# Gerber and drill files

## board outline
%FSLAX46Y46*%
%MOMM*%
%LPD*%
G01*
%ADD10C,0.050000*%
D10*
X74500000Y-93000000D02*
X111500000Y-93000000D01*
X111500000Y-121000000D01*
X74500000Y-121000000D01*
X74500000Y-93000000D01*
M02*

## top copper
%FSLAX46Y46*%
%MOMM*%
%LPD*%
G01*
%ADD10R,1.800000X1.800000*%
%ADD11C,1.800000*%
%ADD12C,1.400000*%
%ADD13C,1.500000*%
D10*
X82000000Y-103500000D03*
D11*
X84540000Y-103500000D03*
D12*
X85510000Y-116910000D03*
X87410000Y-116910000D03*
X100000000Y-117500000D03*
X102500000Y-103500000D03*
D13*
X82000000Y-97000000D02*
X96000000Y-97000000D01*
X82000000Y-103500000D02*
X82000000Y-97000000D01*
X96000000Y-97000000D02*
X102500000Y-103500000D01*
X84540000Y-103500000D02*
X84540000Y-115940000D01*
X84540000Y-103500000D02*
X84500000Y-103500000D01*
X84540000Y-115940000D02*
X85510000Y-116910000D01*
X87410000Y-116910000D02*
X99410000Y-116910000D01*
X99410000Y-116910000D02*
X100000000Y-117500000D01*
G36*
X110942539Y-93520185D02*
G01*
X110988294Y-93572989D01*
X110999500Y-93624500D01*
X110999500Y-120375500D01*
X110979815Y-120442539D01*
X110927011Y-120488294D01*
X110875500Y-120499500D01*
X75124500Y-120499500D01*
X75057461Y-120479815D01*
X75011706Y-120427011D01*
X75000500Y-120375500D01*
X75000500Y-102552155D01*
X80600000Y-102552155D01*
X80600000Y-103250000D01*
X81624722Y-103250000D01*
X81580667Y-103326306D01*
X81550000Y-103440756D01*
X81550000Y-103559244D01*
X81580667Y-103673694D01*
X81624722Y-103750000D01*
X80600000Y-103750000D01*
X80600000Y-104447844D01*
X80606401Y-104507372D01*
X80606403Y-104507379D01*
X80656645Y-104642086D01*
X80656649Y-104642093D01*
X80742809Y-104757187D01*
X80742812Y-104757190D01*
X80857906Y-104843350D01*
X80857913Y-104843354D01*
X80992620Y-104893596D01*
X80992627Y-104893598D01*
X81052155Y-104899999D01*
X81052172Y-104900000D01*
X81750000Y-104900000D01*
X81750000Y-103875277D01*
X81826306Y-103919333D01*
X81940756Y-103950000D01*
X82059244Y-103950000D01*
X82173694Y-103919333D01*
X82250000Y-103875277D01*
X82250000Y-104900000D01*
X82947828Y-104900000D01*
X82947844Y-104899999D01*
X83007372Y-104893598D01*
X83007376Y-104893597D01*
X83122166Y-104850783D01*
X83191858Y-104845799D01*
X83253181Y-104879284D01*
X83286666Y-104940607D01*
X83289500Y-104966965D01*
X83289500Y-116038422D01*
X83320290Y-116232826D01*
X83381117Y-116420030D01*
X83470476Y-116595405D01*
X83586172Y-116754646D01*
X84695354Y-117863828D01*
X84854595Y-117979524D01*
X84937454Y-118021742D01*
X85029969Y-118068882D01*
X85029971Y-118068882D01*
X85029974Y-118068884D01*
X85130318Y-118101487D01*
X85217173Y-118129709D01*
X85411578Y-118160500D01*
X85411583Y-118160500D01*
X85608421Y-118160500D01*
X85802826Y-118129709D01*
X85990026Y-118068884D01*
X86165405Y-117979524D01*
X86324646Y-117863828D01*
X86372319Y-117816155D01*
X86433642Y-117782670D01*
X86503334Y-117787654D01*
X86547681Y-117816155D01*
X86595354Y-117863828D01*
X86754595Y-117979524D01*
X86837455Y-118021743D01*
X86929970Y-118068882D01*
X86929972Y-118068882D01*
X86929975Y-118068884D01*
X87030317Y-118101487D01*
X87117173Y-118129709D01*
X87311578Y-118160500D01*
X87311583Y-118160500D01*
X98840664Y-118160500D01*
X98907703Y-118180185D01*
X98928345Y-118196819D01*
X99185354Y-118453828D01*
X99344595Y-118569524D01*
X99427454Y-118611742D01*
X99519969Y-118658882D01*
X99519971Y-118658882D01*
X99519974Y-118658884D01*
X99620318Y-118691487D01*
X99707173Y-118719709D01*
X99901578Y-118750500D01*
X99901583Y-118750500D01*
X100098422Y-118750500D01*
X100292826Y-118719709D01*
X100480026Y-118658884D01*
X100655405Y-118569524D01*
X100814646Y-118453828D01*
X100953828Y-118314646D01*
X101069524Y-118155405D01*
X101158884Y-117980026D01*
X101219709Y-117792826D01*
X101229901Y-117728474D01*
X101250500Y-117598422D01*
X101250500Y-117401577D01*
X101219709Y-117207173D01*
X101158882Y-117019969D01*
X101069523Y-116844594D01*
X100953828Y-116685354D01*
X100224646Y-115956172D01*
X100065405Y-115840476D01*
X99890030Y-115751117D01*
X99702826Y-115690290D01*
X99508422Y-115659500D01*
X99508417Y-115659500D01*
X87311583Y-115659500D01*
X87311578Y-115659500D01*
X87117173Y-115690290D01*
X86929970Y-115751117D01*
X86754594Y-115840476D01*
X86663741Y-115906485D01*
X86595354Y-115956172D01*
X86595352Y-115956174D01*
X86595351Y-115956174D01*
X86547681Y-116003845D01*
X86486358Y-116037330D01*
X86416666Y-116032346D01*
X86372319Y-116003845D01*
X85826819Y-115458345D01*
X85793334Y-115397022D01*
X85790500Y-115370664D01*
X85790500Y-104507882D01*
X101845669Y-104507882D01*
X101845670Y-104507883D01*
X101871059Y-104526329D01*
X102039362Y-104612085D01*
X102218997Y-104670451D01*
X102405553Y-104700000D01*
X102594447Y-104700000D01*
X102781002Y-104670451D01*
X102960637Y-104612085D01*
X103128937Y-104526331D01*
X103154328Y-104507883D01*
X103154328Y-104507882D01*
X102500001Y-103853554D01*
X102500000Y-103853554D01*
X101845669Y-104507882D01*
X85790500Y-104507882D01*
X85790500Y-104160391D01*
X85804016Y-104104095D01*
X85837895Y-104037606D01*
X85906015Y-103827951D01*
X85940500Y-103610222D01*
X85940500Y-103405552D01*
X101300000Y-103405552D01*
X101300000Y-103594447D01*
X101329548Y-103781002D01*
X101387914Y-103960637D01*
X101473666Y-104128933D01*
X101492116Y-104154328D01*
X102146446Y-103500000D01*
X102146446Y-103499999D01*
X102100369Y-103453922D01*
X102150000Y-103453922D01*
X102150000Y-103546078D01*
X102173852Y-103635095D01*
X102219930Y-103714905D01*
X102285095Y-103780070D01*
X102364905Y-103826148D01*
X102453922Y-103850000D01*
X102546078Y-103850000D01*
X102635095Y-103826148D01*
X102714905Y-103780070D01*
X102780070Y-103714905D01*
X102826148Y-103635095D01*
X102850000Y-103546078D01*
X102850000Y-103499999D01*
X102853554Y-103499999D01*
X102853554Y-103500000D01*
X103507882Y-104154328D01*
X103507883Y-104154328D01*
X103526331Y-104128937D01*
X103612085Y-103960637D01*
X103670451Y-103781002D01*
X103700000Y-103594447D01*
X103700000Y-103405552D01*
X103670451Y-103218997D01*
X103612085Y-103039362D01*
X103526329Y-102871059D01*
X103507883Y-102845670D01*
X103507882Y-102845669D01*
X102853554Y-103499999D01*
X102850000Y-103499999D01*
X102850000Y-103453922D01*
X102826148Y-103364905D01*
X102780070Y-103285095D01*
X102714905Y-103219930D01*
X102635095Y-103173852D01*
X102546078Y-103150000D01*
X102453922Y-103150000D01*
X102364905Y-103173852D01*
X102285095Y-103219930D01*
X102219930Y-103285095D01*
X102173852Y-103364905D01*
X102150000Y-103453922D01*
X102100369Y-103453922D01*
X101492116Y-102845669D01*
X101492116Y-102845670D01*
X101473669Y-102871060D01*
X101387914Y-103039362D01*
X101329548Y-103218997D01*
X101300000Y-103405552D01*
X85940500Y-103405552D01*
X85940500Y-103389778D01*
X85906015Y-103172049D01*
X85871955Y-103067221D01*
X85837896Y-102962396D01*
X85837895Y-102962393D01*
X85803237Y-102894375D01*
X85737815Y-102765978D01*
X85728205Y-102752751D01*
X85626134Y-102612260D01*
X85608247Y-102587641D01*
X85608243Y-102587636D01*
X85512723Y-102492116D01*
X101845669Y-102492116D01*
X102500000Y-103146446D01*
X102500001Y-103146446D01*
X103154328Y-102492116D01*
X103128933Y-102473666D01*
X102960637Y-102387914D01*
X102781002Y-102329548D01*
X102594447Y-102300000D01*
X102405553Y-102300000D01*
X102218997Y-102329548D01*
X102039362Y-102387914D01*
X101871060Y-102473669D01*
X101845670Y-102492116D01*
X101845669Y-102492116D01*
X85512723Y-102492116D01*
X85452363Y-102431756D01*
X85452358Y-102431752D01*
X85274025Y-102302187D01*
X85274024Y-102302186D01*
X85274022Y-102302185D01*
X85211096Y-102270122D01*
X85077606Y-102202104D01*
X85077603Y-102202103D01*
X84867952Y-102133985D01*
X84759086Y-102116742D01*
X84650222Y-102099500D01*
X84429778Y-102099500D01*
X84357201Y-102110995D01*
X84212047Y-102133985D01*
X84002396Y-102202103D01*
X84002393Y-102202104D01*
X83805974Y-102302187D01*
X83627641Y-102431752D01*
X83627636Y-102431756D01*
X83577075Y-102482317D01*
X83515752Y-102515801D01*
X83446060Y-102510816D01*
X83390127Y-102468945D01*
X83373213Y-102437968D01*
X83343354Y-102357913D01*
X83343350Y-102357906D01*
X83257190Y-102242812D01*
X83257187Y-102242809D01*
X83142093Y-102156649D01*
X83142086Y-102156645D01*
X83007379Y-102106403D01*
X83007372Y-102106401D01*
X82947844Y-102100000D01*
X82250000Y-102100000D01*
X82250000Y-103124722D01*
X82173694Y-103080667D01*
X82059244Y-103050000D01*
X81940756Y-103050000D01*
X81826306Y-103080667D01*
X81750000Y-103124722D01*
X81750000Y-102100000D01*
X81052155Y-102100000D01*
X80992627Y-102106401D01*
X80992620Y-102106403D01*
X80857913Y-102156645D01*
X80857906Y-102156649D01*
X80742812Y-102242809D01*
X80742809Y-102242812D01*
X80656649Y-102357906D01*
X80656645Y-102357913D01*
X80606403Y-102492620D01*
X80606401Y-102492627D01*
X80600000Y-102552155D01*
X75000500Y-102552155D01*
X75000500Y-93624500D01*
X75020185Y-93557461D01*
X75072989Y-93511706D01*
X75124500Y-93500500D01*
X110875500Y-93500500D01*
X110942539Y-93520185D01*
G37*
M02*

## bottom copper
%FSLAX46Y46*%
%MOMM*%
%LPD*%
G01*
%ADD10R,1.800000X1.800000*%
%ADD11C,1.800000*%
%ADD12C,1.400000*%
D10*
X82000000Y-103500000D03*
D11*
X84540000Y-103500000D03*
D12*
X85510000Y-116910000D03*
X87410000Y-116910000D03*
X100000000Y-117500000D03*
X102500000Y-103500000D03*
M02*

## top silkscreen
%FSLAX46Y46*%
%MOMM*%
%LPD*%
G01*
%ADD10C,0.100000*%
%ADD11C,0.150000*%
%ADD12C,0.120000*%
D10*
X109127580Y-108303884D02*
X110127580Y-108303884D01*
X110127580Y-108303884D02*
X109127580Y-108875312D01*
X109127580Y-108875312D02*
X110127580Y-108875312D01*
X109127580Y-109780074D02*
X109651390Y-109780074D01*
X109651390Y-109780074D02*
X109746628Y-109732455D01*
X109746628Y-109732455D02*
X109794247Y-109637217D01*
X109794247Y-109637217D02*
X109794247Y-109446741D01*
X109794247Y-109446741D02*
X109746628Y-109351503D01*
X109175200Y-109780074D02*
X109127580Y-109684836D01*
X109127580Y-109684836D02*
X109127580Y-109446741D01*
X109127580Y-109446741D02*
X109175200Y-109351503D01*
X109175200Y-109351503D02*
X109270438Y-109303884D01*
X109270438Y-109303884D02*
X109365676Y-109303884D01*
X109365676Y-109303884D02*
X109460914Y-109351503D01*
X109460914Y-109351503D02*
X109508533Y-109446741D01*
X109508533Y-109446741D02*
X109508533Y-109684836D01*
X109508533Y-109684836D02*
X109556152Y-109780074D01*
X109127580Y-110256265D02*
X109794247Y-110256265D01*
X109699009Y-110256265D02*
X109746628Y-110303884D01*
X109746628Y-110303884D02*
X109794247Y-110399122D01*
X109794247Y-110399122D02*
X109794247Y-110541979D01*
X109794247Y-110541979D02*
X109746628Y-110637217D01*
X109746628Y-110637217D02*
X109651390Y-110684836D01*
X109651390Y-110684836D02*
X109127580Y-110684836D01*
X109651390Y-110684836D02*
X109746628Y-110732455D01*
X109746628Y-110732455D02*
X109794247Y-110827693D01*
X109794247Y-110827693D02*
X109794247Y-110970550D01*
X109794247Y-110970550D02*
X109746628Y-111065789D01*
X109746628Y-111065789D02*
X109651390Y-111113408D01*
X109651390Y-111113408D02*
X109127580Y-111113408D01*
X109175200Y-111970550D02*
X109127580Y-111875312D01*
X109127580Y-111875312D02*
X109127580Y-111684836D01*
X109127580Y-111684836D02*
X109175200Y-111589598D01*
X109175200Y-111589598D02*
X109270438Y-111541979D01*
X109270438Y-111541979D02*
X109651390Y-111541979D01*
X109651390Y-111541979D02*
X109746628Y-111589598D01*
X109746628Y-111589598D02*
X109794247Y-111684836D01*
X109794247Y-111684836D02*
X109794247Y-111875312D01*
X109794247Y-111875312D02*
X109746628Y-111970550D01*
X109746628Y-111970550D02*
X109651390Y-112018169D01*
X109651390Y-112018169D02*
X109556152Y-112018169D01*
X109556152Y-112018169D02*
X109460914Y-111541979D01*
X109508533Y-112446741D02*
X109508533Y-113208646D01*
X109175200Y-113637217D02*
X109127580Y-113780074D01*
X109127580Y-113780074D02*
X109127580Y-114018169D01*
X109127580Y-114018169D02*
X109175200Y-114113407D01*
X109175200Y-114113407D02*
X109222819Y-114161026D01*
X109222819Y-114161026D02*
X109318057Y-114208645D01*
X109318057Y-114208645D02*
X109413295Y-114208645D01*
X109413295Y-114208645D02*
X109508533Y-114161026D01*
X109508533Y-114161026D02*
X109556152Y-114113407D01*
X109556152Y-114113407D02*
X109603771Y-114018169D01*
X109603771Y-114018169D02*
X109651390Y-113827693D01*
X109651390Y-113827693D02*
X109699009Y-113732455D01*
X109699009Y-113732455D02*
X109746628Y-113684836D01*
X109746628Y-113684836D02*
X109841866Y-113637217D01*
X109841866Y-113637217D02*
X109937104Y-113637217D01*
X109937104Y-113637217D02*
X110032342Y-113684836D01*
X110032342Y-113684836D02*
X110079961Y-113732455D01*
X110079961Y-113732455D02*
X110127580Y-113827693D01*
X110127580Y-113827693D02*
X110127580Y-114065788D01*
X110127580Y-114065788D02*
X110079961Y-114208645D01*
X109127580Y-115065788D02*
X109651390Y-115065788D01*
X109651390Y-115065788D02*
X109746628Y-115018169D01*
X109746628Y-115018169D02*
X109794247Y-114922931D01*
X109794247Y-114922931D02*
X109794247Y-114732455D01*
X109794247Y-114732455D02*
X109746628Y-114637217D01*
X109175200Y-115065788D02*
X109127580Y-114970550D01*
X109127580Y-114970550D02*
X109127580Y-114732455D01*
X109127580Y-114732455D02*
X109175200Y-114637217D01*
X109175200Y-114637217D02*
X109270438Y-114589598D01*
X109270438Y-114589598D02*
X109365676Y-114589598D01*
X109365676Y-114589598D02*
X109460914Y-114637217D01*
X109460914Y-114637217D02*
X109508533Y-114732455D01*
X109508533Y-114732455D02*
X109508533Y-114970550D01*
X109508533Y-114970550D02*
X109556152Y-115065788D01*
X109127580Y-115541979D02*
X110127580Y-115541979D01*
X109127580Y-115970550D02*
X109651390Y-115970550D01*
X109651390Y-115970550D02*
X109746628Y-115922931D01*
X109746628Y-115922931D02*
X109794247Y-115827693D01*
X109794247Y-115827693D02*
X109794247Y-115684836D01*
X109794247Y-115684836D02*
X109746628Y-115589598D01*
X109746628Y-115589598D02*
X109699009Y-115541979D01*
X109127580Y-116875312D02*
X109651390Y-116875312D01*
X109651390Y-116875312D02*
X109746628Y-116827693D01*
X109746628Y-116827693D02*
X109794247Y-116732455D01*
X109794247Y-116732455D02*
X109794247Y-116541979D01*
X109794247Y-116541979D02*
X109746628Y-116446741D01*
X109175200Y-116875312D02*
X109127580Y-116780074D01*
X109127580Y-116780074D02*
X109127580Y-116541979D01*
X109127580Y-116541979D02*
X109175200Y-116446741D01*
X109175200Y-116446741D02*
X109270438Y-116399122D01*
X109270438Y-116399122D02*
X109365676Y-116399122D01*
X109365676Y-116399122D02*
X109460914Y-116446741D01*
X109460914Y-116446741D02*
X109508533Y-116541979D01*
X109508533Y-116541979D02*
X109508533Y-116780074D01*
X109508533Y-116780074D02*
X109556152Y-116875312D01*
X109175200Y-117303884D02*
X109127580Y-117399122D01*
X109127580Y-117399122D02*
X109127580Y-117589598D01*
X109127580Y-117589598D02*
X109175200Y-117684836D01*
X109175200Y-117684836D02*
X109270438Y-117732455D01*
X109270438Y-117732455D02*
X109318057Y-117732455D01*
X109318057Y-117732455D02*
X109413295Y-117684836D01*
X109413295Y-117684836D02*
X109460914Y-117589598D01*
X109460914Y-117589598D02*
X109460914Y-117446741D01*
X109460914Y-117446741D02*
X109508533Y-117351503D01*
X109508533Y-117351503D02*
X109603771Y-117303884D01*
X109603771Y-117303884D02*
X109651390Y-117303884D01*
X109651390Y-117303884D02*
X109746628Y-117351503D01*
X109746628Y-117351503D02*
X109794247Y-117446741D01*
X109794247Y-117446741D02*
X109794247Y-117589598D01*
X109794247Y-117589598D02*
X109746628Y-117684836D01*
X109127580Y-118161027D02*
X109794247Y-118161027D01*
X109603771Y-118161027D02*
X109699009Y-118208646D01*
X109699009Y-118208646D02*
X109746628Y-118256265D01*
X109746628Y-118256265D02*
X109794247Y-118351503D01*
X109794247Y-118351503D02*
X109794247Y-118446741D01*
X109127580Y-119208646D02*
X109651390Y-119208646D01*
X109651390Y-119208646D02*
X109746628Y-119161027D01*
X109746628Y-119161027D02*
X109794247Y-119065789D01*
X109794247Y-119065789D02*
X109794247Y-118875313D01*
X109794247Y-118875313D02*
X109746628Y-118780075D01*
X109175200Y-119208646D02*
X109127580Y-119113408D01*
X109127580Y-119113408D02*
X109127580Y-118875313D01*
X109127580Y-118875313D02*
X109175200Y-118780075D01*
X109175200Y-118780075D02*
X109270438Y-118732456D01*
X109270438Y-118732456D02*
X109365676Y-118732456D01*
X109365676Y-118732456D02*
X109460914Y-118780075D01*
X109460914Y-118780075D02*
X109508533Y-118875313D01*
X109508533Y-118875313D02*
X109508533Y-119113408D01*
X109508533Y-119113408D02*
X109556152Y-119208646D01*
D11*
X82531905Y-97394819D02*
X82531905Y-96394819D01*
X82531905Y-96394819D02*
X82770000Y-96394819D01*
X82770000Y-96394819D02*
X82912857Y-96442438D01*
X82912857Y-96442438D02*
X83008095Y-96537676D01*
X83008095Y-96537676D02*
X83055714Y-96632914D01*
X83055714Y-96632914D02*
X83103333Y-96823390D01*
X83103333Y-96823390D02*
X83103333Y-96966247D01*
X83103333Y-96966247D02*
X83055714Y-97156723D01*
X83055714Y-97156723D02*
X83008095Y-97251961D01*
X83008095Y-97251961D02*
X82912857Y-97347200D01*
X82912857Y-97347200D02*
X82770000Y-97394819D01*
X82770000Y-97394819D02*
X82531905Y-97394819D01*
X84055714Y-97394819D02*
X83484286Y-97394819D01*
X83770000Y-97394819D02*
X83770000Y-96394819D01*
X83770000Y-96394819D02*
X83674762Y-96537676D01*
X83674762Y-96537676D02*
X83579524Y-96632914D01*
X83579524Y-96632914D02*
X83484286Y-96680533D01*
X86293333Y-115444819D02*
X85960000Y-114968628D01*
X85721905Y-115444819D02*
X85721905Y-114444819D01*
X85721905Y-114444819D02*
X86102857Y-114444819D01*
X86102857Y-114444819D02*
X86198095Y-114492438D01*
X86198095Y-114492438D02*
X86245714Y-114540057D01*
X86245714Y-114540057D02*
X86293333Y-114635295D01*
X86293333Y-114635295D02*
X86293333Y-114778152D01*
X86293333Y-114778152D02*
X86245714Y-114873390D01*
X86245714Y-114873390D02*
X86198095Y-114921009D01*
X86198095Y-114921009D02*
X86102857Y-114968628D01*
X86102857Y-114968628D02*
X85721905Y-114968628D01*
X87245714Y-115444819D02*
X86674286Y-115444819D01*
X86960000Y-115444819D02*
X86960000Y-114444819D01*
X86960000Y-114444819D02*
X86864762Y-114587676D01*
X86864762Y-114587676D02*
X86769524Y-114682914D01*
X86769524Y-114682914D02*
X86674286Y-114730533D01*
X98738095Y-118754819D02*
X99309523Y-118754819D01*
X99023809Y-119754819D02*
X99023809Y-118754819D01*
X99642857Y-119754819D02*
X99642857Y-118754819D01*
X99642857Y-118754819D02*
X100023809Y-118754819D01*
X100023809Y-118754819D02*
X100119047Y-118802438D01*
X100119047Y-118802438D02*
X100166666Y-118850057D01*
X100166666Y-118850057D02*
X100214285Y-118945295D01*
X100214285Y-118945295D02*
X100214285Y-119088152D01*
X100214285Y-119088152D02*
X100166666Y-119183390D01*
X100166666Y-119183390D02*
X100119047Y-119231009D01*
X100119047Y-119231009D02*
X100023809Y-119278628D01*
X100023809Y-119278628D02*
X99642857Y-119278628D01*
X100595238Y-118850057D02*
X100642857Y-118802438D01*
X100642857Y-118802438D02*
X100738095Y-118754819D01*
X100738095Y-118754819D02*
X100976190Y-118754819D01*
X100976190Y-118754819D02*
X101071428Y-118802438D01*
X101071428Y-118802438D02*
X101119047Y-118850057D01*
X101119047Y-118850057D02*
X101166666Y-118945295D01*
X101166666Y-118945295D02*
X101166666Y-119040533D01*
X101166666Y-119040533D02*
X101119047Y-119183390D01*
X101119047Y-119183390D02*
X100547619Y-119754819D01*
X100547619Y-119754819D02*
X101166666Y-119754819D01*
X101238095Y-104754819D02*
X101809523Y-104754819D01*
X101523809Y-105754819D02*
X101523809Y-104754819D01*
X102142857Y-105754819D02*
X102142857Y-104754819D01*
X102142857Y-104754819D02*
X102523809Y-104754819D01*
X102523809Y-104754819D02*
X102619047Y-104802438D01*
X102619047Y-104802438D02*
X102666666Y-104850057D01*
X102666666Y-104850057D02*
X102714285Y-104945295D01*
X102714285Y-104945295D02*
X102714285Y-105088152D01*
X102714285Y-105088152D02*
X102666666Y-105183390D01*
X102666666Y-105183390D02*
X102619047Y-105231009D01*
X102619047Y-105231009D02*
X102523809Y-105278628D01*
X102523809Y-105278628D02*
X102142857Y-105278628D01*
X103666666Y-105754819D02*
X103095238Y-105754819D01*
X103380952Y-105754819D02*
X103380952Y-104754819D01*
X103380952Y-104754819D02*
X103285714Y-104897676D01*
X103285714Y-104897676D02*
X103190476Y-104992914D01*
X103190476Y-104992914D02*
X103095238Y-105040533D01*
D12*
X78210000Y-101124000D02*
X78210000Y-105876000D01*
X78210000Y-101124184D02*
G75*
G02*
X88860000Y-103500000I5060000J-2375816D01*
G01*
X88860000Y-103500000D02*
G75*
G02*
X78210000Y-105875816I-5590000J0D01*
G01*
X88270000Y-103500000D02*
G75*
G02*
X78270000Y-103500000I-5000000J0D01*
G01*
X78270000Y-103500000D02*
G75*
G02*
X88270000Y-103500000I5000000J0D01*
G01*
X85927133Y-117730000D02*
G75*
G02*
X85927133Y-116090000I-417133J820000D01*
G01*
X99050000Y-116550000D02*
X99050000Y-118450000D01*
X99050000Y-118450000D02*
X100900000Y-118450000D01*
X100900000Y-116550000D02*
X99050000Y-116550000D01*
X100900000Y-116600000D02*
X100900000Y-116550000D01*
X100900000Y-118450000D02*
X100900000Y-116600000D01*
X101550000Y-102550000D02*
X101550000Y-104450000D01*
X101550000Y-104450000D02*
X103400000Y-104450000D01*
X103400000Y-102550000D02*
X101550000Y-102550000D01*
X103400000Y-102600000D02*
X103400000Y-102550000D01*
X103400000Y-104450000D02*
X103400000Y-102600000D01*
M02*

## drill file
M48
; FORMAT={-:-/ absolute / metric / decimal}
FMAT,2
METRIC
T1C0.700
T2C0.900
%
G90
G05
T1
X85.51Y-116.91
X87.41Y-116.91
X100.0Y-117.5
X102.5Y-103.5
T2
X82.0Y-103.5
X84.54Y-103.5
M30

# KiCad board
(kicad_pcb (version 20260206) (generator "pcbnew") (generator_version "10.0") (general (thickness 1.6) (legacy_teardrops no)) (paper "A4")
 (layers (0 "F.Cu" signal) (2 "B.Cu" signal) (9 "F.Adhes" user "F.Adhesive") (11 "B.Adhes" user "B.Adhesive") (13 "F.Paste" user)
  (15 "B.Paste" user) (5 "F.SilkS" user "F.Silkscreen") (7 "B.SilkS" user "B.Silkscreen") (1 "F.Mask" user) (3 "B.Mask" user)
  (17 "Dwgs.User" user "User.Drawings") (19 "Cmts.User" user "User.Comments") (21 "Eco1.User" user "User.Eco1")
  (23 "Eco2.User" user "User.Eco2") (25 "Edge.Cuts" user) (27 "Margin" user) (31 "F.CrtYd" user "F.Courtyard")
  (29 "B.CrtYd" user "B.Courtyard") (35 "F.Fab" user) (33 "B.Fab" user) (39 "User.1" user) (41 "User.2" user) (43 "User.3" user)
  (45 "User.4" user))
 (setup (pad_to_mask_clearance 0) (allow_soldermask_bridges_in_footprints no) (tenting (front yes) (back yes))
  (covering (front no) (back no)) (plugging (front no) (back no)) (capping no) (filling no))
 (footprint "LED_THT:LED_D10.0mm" (layer "F.Cu") (at 82 103.5)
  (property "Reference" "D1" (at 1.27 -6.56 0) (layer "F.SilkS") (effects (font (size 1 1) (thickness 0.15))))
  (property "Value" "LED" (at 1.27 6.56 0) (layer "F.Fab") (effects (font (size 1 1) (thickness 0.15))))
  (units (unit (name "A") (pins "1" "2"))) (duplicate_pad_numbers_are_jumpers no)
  (fp_line (start -3.79 -2.376) (end -3.79 2.376) (stroke (width 0.12) (type solid)) (layer "F.SilkS"))
  (fp_arc (start -3.79 -2.375816) (mid 2.487107 -5.455891) (end 6.86 0) (stroke (width 0.12) (type solid)) (layer "F.SilkS"))
  (fp_arc (start 6.86 0) (mid 2.487107 5.455891) (end -3.79 2.375816) (stroke (width 0.12) (type solid)) (layer "F.SilkS"))
  (fp_circle (center 1.27 0) (end 6.27 0) (stroke (width 0.12) (type solid)) (fill no) (layer "F.SilkS"))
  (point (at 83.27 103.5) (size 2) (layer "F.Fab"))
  (pad "1" thru_hole rect (at 0 0) (size 1.8 1.8) (drill 0.9) (layers "*.Cu" "*.Mask") (remove_unused_layers no) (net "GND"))
  (pad "2" thru_hole circle (at 2.54 0) (size 1.8 1.8) (drill 0.9) (layers "*.Cu" "*.Mask") (remove_unused_layers no) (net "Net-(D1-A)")))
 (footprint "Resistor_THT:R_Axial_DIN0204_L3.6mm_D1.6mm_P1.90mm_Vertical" (layer "F.Cu") (at 85.51 116.91)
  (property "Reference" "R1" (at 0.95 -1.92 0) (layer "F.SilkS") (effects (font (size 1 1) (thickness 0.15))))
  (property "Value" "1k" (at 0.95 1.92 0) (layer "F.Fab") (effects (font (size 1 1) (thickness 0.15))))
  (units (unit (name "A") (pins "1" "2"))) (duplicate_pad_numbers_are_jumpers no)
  (fp_arc (start 0.417133 0.82) (mid -0.92 0) (end 0.417133 -0.82) (stroke (width 0.12) (type solid)) (layer "F.SilkS"))
  (pad "1" thru_hole circle (at 0 0) (size 1.4 1.4) (drill 0.7) (layers "*.Cu" "*.Mask") (remove_unused_layers no) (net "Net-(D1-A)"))
  (pad "2" thru_hole circle (at 1.9 0) (size 1.4 1.4) (drill 0.7) (layers "*.Cu" "*.Mask") (remove_unused_layers no) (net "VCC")))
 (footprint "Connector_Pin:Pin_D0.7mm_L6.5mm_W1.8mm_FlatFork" (layer "F.Cu") (at 100 117.5)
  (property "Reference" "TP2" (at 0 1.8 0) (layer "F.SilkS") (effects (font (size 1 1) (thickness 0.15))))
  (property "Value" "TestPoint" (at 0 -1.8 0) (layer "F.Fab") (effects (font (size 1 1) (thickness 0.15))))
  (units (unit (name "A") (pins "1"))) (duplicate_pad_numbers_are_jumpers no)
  (fp_line (start -0.95 -0.95) (end -0.95 0.95) (stroke (width 0.12) (type solid)) (layer "F.SilkS"))
  (fp_line (start -0.95 0.95) (end 0.9 0.95) (stroke (width 0.12) (type solid)) (layer "F.SilkS"))
  (fp_line (start 0.9 -0.95) (end -0.95 -0.95) (stroke (width 0.12) (type solid)) (layer "F.SilkS"))
  (fp_line (start 0.9 -0.9) (end 0.9 -0.95) (stroke (width 0.12) (type solid)) (layer "F.SilkS"))
  (fp_line (start 0.9 0.95) (end 0.9 -0.9) (stroke (width 0.12) (type solid)) (layer "F.SilkS"))
  (pad "1" thru_hole circle (at 0 0) (size 1.4 1.4) (drill 0.7) (layers "*.Cu" "*.Mask") (remove_unused_layers no) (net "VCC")))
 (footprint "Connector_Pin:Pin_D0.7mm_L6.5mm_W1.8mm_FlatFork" (layer "F.Cu") (at 102.5 103.5)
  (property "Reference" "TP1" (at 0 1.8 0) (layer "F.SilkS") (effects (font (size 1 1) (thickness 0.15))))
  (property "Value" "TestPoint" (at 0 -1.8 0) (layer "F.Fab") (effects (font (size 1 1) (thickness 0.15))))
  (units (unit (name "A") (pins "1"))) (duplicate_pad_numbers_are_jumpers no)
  (fp_line (start -0.95 -0.95) (end -0.95 0.95) (stroke (width 0.12) (type solid)) (layer "F.SilkS"))
  (fp_line (start -0.95 0.95) (end 0.9 0.95) (stroke (width 0.12) (type solid)) (layer "F.SilkS"))
  (fp_line (start 0.9 -0.95) (end -0.95 -0.95) (stroke (width 0.12) (type solid)) (layer "F.SilkS"))
  (fp_line (start 0.9 -0.9) (end 0.9 -0.95) (stroke (width 0.12) (type solid)) (layer "F.SilkS"))
  (fp_line (start 0.9 0.95) (end 0.9 -0.9) (stroke (width 0.12) (type solid)) (layer "F.SilkS"))
  (pad "1" thru_hole circle (at 0 0) (size 1.4 1.4) (drill 0.7) (layers "*.Cu" "*.Mask") (remove_unused_layers no) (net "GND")))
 (gr_rect (start 74.5 93) (end 111.5 121) (stroke (width 0.05) (type default)) (fill no) (layer "Edge.Cuts"))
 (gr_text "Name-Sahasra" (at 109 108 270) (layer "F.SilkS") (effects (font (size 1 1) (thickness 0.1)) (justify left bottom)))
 (segment (start 82 97) (end 96 97) (width 1.5) (layer "F.Cu") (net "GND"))
 (segment (start 82 103.5) (end 82 97) (width 1.5) (layer "F.Cu") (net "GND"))
 (segment (start 96 97) (end 102.5 103.5) (width 1.5) (layer "F.Cu") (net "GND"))
 (segment (start 84.54 103.5) (end 84.54 115.94) (width 1.5) (layer "F.Cu") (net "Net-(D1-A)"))
 (segment (start 84.54 103.5) (end 84.5 103.5) (width 1.5) (layer "F.Cu") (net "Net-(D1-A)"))
 (segment (start 84.54 115.94) (end 85.51 116.91) (width 1.5) (layer "F.Cu") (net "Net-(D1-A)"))
 (segment (start 87.41 116.91) (end 99.41 116.91) (width 1.5) (layer "F.Cu") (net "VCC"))
 (segment (start 99.41 116.91) (end 100 117.5) (width 1.5) (layer "F.Cu") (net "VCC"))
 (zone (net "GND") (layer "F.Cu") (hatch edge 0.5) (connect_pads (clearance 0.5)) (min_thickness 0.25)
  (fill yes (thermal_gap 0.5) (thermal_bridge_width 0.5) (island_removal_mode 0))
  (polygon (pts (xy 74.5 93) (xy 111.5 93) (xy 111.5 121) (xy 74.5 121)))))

